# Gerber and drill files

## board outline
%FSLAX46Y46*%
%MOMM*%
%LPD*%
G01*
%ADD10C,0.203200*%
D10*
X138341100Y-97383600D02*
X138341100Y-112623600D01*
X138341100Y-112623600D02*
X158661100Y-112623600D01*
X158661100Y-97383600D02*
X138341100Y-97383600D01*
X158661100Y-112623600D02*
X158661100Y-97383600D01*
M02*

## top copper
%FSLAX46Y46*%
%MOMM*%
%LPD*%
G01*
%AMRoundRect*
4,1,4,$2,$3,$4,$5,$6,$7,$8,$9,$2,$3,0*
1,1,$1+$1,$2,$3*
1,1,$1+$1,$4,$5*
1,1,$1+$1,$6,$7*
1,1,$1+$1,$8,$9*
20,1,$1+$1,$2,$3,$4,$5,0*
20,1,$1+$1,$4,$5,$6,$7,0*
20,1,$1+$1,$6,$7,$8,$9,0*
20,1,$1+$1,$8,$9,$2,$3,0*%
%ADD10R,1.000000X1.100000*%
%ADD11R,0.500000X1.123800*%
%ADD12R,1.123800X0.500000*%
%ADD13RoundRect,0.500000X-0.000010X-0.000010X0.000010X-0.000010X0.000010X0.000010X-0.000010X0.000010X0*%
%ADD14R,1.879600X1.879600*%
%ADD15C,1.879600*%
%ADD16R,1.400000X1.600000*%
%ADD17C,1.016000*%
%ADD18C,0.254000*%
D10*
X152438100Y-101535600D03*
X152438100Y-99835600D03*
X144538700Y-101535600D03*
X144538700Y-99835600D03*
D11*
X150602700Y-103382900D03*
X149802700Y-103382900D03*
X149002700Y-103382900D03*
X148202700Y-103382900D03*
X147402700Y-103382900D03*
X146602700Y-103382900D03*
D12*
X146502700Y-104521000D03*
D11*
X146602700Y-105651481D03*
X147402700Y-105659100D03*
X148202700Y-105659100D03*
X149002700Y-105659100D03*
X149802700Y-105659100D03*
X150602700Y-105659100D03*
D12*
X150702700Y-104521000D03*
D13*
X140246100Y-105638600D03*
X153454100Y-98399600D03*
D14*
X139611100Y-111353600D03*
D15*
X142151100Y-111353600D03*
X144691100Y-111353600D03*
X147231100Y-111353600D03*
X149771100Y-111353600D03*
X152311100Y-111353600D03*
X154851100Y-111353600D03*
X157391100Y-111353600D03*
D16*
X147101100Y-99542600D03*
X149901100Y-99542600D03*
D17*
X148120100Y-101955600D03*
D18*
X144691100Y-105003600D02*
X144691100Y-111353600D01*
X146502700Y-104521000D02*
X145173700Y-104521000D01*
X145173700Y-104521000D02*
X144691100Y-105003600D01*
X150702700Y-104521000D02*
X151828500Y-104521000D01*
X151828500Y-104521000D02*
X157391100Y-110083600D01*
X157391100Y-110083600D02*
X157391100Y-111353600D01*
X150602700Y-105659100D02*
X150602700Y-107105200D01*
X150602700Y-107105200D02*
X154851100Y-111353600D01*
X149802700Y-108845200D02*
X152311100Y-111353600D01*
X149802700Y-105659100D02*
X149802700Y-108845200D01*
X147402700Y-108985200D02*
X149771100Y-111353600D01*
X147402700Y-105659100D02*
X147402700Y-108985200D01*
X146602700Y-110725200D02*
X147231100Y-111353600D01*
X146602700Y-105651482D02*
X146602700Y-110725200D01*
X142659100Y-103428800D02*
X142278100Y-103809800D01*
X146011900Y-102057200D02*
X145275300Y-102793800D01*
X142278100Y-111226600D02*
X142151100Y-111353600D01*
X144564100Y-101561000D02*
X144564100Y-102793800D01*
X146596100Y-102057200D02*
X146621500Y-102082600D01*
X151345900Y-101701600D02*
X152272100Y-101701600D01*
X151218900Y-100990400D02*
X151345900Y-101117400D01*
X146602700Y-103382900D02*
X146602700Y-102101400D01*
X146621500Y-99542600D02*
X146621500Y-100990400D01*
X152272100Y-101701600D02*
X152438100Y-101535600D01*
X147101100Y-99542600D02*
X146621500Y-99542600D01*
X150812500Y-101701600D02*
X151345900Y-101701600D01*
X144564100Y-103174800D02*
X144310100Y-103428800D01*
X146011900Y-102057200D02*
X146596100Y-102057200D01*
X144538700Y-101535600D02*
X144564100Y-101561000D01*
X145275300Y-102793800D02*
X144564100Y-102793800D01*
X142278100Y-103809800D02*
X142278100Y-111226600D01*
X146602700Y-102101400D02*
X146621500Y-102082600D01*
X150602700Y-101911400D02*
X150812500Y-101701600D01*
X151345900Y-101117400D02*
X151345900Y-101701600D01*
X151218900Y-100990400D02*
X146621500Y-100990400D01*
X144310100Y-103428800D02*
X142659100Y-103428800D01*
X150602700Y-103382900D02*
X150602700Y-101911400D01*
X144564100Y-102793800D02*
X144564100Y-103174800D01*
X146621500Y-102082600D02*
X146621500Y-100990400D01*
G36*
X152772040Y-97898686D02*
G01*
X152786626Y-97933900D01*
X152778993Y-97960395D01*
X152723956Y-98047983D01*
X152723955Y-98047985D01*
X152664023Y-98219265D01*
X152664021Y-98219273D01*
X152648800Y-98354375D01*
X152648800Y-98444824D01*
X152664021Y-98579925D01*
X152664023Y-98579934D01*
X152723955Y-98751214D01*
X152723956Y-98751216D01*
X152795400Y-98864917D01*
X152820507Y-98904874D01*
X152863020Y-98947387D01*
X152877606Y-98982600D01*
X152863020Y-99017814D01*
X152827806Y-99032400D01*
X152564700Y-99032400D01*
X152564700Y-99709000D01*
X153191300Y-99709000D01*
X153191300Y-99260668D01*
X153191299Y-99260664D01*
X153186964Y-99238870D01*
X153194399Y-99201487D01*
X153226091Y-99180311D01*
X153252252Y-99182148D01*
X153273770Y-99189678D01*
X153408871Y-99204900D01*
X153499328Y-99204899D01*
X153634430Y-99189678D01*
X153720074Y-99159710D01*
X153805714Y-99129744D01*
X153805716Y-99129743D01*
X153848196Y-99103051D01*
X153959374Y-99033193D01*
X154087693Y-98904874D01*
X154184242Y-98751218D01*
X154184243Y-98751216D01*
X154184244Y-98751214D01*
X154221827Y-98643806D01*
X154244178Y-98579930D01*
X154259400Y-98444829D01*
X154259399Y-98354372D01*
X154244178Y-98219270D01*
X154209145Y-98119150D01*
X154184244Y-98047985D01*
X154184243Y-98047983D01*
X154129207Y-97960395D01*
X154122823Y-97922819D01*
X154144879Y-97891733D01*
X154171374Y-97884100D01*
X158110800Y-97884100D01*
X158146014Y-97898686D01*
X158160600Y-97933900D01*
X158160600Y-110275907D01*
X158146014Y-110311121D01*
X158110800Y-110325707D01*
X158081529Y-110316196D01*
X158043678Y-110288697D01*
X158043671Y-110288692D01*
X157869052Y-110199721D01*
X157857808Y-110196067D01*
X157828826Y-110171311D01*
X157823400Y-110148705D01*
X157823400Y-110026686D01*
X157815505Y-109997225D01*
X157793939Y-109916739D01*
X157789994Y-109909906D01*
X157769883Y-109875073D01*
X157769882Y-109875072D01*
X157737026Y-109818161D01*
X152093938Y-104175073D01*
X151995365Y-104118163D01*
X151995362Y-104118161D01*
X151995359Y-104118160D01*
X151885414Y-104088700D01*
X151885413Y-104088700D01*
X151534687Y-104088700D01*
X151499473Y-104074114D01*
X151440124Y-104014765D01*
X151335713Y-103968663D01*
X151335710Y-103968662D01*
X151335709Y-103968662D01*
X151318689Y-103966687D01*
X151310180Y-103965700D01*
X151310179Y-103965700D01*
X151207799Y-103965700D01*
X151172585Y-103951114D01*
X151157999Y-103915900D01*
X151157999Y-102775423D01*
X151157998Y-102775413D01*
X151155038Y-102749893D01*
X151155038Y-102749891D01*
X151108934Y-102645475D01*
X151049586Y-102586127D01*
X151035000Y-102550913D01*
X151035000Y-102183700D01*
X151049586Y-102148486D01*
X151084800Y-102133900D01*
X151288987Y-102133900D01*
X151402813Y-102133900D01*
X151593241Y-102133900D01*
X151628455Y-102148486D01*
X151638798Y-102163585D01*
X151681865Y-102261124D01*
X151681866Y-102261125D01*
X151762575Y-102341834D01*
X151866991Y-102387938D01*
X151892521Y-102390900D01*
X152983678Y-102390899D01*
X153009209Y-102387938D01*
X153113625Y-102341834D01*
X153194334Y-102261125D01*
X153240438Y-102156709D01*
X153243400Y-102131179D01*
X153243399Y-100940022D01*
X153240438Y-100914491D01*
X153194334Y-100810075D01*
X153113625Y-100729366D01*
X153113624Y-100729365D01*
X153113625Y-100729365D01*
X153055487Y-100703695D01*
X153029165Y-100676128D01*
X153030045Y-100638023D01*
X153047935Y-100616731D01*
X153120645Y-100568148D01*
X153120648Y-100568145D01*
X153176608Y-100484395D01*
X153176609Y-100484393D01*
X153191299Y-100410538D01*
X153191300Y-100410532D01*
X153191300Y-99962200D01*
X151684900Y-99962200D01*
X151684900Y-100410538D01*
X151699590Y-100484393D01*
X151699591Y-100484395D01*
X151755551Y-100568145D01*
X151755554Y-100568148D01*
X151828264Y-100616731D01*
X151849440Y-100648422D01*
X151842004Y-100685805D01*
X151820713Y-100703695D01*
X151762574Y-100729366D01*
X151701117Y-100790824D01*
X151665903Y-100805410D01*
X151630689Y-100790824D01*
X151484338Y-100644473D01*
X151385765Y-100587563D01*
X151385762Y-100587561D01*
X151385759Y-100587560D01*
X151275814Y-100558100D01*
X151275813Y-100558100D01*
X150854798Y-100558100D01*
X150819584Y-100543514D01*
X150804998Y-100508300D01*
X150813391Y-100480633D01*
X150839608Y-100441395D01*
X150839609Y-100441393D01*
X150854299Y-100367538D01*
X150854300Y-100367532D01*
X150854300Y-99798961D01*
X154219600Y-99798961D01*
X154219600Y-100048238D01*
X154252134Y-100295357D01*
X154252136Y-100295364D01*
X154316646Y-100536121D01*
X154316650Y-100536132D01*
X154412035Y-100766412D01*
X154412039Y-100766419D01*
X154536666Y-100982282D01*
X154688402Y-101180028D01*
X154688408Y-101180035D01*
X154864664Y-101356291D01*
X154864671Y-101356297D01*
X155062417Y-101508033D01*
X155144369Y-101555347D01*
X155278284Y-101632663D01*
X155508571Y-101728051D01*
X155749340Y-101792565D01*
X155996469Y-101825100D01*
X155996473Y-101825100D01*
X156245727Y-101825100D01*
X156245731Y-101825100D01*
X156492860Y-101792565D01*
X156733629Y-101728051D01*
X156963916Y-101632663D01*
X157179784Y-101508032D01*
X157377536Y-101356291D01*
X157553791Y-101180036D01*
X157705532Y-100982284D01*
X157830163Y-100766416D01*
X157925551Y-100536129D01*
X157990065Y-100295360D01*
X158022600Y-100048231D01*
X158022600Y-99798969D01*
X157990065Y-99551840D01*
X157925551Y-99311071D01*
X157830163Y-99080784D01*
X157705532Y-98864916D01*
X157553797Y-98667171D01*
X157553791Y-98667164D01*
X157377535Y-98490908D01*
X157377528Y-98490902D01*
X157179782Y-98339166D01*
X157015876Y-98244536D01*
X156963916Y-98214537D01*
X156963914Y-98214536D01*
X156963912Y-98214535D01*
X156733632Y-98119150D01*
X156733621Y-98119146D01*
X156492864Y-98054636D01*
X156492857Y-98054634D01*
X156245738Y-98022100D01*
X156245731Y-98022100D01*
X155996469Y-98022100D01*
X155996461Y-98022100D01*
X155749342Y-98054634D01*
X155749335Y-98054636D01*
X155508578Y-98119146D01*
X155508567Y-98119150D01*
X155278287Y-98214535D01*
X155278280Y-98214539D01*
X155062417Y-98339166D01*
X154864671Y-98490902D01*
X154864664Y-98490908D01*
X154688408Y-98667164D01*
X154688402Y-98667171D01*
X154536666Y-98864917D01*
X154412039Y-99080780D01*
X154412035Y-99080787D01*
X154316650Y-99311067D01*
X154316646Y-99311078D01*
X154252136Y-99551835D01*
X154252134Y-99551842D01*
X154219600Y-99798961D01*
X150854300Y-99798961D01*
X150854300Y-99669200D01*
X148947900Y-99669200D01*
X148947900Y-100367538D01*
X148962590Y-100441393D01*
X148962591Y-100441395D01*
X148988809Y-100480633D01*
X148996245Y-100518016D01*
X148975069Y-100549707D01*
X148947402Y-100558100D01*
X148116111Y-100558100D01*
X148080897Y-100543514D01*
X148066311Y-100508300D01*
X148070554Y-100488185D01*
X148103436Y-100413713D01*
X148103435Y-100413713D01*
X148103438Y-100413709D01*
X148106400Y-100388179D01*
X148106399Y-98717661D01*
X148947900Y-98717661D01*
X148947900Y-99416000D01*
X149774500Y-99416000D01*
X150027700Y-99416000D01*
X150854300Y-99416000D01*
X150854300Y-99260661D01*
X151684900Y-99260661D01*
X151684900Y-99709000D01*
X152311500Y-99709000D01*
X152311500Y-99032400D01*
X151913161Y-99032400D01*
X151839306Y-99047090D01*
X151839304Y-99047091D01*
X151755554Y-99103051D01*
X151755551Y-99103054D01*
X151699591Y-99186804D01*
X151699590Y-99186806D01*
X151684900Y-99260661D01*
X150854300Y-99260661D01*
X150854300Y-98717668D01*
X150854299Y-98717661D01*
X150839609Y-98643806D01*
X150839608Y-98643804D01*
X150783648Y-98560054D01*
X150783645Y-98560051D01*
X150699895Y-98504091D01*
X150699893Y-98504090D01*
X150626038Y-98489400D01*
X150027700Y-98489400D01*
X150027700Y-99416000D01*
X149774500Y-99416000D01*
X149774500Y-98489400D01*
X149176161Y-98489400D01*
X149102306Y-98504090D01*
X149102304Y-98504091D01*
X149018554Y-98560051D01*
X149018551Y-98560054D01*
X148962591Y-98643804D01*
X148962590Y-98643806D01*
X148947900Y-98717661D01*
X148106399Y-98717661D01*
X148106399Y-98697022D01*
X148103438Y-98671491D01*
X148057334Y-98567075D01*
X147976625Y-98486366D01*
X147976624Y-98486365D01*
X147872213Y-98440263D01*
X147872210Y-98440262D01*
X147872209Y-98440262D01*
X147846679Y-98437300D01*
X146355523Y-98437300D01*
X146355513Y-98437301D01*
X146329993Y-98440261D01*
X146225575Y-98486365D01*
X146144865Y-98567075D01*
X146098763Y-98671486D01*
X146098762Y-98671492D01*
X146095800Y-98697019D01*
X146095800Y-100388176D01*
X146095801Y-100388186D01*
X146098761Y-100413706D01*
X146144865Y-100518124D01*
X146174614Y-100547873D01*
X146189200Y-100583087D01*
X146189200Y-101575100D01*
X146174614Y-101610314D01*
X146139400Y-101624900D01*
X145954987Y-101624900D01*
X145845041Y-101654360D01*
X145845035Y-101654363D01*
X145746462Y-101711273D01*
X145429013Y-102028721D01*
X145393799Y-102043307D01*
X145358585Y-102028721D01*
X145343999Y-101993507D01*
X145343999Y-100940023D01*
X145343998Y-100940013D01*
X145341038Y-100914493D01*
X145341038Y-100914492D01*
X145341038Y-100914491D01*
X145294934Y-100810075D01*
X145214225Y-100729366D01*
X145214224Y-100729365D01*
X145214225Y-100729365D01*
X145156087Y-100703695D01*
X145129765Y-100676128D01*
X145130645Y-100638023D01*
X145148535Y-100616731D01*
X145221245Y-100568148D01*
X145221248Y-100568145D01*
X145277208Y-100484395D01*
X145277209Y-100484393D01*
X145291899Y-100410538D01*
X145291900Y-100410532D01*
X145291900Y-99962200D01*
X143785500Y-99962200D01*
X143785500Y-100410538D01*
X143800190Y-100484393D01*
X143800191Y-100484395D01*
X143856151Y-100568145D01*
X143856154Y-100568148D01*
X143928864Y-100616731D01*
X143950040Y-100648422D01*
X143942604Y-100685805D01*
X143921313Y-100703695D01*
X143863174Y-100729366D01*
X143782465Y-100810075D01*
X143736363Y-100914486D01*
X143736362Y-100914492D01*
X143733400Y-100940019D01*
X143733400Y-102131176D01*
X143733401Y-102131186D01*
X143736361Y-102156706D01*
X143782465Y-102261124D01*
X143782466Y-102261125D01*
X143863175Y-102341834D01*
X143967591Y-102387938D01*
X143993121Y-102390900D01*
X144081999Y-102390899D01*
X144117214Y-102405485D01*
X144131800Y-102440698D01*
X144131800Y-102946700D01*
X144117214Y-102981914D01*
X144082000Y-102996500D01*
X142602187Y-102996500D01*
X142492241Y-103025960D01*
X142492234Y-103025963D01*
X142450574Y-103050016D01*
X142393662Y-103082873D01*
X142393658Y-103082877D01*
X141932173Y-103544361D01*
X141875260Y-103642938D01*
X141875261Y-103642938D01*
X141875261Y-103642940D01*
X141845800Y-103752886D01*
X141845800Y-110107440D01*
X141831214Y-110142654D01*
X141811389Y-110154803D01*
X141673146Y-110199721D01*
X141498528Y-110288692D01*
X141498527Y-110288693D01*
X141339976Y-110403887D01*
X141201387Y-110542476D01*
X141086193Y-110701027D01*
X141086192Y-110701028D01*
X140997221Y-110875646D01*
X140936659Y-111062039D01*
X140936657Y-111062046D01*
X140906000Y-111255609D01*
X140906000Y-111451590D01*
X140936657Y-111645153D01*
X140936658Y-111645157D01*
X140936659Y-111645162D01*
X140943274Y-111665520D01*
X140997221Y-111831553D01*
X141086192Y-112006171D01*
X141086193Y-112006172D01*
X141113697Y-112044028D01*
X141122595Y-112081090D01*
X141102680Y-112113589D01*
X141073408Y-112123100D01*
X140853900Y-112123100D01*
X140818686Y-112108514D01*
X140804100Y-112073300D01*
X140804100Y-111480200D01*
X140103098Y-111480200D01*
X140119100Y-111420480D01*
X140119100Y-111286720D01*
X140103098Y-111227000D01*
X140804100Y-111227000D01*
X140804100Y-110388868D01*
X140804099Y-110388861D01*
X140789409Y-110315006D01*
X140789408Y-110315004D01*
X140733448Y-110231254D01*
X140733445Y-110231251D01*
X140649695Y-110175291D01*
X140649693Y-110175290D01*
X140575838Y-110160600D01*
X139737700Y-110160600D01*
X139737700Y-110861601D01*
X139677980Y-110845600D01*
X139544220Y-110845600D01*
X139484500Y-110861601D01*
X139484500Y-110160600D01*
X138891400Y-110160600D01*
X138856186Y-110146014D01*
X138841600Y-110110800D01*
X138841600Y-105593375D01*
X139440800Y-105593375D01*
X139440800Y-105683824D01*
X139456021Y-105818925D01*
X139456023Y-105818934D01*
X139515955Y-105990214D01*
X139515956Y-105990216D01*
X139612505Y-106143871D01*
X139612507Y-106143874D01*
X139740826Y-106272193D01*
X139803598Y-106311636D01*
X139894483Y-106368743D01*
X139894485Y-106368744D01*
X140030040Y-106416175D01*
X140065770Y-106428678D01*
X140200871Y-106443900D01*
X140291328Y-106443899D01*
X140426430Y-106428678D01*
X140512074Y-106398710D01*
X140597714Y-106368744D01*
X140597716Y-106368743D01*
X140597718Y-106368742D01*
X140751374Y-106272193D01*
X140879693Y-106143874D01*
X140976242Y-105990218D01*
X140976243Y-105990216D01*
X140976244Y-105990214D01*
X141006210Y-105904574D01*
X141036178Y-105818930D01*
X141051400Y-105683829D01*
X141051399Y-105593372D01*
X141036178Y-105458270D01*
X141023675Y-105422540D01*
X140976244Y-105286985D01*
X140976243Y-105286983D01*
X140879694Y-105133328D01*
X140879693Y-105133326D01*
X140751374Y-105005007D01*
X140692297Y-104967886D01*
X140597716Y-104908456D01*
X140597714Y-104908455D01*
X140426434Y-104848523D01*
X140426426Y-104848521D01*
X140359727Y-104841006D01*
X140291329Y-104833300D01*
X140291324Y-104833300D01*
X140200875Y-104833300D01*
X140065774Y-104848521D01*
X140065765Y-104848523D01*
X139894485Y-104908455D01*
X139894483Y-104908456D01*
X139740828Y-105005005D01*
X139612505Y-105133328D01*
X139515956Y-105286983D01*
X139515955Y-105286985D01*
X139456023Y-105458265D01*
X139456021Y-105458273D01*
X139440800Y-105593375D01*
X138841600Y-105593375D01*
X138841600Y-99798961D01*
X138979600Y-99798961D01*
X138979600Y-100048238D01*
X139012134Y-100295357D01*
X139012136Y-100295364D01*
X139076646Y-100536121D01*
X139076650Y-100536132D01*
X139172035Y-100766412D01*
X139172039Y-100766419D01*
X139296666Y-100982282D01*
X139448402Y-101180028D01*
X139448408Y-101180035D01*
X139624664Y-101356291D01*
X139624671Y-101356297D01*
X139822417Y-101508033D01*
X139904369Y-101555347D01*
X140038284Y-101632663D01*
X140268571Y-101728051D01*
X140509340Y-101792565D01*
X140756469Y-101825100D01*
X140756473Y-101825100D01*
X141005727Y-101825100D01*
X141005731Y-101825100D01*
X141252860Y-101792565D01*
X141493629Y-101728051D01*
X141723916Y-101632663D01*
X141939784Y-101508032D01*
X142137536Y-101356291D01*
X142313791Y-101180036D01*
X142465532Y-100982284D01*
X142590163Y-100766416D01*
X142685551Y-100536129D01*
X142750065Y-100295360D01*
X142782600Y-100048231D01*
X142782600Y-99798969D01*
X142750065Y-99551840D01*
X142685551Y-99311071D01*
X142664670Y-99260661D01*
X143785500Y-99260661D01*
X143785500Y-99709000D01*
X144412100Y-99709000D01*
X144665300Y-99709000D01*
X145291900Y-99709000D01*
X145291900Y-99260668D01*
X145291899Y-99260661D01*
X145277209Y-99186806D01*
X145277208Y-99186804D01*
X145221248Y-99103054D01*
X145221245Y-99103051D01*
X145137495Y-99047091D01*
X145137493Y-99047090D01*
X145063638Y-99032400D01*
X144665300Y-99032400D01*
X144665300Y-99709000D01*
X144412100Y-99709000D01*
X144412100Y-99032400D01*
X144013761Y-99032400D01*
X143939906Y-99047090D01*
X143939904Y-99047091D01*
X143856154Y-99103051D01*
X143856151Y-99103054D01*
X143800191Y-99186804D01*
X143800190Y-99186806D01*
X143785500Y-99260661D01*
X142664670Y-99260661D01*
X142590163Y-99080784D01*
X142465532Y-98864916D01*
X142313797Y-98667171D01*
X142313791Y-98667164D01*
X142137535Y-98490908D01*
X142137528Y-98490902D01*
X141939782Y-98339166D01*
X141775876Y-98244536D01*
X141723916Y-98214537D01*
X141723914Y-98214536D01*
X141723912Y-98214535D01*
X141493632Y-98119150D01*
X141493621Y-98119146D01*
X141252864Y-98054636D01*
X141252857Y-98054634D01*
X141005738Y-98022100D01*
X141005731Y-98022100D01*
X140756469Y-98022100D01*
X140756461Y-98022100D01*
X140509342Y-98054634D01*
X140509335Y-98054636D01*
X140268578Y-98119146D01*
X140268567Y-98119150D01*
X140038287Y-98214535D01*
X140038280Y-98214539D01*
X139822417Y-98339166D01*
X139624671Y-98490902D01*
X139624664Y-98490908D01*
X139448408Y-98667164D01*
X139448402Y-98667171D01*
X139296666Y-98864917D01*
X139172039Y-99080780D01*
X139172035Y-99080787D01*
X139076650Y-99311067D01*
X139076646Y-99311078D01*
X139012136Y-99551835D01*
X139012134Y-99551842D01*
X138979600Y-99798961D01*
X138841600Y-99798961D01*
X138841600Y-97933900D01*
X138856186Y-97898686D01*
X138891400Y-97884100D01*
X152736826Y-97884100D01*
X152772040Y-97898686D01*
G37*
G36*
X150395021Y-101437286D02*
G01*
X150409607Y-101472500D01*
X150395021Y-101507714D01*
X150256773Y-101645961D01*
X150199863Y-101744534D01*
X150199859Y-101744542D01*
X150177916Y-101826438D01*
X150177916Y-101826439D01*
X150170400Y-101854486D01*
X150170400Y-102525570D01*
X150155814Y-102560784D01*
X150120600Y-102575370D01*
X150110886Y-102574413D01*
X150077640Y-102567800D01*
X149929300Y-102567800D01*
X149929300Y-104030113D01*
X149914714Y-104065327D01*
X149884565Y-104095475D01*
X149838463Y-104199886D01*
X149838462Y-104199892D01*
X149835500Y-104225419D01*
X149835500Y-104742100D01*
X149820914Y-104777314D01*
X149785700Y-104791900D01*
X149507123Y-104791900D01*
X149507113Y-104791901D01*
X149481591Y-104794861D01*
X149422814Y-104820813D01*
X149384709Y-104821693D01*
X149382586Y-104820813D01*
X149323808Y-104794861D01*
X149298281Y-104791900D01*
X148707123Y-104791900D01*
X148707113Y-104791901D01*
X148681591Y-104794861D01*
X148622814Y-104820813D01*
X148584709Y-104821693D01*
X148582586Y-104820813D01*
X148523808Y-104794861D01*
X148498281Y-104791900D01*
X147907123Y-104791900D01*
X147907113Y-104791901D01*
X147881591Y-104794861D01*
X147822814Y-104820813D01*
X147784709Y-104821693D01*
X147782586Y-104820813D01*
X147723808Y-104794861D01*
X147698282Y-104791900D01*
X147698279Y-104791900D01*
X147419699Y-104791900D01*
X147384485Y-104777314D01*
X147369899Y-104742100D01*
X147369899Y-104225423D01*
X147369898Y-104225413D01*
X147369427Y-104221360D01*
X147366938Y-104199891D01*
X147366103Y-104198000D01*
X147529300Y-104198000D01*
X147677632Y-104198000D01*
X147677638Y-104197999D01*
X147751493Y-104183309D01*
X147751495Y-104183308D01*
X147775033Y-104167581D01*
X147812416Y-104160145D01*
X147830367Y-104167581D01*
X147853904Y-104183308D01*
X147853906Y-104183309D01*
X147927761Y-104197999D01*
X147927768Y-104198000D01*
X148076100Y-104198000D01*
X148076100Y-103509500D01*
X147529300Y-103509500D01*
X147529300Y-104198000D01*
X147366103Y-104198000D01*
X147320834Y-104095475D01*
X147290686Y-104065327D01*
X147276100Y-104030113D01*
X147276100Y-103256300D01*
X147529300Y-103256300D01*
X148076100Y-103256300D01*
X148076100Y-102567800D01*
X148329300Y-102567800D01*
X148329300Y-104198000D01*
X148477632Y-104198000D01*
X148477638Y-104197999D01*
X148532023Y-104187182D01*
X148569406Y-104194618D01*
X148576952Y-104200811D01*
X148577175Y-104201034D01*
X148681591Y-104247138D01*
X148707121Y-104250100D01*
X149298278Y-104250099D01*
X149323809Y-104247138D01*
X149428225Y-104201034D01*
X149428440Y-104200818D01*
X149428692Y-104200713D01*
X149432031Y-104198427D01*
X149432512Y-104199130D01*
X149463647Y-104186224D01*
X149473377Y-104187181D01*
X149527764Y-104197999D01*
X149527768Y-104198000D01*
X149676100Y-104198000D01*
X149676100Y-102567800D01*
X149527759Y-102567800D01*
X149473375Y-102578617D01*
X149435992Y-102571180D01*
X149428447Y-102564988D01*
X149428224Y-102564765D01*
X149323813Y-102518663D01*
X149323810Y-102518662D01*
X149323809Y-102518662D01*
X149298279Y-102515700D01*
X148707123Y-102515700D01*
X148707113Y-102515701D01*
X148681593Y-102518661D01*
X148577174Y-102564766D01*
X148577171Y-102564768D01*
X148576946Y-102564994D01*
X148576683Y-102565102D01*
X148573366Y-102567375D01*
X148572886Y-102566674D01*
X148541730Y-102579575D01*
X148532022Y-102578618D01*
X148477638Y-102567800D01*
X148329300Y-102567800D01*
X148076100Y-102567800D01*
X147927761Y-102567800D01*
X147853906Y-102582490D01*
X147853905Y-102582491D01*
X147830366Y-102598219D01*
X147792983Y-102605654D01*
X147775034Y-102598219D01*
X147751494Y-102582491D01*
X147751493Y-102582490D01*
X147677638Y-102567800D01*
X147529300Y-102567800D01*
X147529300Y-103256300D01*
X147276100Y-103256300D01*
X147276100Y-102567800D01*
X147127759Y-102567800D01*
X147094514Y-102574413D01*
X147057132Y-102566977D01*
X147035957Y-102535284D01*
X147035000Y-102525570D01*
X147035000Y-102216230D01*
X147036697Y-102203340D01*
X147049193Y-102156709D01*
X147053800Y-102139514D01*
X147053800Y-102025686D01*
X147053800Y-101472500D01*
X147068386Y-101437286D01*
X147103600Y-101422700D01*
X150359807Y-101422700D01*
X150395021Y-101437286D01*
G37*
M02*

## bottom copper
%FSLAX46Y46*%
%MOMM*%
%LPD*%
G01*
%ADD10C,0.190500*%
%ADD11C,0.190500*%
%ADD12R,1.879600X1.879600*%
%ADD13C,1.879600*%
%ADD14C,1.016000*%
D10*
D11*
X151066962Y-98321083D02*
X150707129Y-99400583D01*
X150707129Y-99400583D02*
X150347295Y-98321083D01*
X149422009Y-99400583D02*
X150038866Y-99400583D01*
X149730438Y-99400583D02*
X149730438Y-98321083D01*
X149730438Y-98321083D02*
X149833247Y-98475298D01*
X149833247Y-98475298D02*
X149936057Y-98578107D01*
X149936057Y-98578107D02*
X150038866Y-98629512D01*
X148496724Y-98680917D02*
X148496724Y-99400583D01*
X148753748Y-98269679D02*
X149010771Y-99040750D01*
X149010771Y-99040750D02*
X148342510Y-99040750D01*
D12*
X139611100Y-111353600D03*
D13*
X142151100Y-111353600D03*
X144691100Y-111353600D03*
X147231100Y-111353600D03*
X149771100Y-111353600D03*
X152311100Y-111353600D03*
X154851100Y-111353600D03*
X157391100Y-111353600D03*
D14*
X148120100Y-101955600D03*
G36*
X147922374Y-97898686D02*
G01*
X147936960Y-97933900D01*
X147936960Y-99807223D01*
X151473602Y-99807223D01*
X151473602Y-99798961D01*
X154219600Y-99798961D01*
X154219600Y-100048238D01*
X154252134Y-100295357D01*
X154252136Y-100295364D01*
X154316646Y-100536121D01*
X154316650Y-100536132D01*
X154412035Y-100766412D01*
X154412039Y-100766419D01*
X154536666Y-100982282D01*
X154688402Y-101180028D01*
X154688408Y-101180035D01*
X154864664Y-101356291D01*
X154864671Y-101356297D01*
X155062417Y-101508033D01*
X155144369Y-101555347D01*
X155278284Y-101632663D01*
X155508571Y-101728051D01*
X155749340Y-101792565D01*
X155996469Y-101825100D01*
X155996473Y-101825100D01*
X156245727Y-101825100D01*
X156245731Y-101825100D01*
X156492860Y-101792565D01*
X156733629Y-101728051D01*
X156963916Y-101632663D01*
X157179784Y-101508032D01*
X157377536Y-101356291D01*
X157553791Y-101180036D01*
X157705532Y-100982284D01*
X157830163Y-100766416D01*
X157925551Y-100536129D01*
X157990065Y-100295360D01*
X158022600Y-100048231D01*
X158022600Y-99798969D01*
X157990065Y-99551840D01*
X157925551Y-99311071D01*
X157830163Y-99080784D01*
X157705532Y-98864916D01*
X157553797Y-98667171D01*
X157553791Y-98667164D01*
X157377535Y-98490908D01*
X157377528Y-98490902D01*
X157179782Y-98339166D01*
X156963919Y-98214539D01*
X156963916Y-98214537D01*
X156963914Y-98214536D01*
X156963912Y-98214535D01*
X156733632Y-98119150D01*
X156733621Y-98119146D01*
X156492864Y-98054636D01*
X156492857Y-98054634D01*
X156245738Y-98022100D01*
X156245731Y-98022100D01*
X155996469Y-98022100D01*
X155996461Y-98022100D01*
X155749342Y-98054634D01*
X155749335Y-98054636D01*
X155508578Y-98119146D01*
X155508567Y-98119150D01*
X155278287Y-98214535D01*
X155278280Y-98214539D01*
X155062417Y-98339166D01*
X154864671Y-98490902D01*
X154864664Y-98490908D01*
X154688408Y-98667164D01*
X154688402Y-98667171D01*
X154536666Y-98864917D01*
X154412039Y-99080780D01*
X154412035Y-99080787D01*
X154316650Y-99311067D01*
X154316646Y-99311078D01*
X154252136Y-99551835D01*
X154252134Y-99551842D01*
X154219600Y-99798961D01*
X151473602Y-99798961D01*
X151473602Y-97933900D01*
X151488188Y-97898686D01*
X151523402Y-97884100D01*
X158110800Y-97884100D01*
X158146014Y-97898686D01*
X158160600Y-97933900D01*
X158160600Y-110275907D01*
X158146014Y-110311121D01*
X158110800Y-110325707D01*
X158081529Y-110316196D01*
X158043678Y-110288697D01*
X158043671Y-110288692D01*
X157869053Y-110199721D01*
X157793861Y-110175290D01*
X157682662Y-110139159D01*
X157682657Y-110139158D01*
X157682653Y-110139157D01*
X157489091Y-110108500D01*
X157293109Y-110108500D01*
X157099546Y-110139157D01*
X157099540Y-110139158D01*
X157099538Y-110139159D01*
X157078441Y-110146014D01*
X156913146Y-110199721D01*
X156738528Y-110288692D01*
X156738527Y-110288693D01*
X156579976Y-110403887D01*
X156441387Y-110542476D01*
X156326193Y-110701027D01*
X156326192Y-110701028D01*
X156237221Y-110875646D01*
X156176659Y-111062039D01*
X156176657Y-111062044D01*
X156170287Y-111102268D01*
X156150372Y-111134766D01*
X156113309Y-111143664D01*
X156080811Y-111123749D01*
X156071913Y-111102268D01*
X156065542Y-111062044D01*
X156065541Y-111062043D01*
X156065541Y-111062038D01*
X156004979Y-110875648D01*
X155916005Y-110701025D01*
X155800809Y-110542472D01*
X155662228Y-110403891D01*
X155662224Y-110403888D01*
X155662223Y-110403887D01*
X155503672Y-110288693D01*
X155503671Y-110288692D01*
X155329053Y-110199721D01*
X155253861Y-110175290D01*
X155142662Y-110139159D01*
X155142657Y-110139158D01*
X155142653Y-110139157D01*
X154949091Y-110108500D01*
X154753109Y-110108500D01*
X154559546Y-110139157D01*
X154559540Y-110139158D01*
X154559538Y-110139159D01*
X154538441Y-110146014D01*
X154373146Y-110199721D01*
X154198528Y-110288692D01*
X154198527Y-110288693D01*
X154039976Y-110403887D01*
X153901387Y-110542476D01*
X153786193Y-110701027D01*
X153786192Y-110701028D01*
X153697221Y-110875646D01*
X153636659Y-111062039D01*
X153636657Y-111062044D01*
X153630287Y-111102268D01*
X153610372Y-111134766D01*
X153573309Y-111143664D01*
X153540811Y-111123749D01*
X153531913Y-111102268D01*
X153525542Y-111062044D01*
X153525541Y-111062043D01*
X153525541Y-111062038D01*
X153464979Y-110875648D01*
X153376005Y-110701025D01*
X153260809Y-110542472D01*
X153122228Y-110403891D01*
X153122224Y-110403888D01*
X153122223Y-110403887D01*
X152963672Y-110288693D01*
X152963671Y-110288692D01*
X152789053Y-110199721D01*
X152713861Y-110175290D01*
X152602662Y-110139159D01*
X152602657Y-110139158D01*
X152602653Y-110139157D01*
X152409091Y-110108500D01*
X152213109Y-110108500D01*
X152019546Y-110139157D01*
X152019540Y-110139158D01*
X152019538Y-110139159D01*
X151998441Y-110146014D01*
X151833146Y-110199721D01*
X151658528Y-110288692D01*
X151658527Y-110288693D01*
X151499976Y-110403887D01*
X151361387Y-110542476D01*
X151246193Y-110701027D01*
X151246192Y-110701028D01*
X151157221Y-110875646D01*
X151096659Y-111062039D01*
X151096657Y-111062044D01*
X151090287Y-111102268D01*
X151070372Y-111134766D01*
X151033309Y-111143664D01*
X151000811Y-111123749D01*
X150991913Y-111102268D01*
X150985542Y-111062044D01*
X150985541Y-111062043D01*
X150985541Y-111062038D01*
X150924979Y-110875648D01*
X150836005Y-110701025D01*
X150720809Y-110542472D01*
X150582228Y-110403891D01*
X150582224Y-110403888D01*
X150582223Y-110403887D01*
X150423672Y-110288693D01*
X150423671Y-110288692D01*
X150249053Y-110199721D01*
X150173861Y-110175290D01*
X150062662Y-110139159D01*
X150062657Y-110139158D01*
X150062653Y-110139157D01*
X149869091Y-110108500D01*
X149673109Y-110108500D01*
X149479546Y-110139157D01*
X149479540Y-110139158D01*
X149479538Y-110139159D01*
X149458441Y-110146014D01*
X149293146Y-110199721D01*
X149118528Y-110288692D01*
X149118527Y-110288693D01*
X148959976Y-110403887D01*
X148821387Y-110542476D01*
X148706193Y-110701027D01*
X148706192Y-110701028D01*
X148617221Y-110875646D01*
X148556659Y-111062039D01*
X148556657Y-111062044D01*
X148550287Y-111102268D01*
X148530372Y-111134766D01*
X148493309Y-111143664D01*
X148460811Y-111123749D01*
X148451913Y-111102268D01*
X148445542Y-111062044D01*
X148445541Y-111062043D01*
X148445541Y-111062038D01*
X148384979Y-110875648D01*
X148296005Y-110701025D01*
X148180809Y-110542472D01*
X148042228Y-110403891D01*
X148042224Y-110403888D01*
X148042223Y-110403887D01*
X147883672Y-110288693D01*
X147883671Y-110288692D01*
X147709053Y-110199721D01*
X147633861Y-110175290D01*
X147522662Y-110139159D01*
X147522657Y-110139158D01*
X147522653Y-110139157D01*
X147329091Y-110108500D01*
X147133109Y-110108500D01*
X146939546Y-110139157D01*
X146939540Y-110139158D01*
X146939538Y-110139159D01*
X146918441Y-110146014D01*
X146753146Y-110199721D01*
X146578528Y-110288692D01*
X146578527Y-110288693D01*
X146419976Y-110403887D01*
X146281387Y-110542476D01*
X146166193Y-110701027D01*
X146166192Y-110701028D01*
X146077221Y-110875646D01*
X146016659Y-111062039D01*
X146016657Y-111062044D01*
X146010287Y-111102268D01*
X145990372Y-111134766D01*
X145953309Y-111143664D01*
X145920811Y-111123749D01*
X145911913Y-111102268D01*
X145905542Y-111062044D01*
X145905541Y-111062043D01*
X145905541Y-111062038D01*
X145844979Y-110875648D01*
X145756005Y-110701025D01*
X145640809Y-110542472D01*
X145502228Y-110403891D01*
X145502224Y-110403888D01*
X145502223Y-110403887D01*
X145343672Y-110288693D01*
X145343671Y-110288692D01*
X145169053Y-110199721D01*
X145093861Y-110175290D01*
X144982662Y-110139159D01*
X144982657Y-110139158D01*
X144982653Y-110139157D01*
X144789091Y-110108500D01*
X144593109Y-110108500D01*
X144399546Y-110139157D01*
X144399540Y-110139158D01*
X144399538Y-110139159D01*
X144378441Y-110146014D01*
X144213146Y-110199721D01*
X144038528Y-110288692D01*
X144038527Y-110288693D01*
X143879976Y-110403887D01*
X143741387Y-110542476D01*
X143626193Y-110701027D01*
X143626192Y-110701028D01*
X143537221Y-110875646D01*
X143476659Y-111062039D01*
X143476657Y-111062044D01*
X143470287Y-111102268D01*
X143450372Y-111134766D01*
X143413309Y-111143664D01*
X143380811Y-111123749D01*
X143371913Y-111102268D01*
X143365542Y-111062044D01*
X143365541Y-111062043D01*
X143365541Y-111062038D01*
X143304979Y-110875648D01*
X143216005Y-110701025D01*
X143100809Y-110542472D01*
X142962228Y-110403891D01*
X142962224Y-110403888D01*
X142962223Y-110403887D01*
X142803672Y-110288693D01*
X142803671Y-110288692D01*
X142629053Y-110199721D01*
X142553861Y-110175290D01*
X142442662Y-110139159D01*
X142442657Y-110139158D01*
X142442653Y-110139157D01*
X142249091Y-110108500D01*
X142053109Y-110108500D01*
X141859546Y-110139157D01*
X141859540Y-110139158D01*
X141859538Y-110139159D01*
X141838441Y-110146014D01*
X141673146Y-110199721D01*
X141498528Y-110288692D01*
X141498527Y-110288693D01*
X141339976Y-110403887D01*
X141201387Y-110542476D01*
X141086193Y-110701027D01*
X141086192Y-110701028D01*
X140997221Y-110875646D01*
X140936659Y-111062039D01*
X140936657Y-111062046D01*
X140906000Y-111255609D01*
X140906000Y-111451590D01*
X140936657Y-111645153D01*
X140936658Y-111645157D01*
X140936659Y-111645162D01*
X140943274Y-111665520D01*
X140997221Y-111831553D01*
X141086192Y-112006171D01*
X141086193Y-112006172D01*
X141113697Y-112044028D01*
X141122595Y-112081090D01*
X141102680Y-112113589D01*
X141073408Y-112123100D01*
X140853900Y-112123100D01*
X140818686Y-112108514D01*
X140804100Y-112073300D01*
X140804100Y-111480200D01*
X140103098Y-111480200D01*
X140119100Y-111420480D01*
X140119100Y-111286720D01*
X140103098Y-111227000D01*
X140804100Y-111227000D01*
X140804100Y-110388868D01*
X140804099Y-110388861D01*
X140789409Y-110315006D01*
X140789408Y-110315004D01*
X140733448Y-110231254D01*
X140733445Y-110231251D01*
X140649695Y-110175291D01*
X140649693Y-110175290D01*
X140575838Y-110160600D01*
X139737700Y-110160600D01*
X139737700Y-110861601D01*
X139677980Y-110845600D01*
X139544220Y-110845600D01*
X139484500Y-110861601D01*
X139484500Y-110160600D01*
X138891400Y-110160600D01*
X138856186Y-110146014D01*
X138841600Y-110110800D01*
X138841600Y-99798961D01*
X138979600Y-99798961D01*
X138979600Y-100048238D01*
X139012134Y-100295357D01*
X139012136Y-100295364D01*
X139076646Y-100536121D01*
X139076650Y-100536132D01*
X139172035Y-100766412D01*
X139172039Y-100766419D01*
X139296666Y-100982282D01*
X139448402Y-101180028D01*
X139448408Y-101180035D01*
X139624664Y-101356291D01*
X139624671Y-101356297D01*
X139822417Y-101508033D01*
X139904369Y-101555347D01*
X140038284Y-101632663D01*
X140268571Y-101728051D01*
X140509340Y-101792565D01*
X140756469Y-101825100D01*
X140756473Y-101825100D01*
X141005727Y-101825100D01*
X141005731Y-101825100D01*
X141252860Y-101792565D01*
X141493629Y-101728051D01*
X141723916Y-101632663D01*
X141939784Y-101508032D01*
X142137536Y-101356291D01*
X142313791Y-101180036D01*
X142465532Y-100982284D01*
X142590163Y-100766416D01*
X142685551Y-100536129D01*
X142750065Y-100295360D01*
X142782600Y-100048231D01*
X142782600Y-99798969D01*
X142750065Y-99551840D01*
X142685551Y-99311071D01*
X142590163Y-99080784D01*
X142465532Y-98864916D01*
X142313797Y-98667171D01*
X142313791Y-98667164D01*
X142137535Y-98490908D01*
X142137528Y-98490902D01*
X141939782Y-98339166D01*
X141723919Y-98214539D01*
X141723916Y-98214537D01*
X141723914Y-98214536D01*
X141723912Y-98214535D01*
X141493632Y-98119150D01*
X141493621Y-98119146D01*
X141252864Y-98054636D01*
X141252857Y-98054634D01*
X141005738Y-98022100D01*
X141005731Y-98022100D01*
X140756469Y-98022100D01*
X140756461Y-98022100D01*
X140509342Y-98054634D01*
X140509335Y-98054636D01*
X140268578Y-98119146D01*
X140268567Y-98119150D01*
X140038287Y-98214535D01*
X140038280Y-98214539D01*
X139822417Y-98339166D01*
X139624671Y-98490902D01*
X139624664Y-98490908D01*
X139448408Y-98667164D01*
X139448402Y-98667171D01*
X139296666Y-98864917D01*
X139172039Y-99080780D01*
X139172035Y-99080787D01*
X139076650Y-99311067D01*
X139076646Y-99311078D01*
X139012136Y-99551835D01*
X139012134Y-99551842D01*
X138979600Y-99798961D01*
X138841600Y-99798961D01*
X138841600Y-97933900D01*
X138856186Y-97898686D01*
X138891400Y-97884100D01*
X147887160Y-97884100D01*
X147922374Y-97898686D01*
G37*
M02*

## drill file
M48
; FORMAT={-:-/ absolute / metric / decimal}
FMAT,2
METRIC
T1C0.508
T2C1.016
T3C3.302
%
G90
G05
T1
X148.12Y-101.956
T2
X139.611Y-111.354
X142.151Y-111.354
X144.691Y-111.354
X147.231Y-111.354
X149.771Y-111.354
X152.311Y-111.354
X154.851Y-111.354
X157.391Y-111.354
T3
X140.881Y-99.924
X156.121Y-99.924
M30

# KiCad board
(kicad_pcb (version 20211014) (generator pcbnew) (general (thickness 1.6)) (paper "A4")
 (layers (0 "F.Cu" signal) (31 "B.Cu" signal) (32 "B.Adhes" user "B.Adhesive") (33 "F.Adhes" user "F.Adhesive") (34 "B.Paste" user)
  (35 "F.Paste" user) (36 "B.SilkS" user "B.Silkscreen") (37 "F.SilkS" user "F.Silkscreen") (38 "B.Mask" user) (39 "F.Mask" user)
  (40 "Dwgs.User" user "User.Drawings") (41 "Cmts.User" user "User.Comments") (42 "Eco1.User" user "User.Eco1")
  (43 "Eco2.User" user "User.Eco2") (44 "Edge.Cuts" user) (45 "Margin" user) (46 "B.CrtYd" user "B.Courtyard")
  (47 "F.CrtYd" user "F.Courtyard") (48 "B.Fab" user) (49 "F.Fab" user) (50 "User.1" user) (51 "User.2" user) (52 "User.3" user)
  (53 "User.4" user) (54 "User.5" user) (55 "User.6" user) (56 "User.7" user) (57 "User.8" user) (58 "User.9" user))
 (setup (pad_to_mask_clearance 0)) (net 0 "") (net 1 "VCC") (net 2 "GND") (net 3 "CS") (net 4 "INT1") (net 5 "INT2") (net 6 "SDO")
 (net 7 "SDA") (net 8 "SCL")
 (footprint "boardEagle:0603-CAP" (layer "F.Cu") (at 152.4381 100.6856 90)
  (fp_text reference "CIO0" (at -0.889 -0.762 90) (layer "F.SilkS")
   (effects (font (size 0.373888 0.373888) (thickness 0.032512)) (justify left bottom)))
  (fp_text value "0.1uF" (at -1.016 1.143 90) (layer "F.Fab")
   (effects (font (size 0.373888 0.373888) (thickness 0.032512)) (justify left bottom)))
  (pad "1" smd rect (at -0.85 0 90) (size 1.1 1) (layers "F.Cu" "F.Paste" "F.Mask") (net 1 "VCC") (solder_mask_margin 0.1016))
  (pad "2" smd rect (at 0.85 0 90) (size 1.1 1) (layers "F.Cu" "F.Paste" "F.Mask") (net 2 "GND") (solder_mask_margin 0.1016)))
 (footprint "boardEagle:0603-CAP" (layer "F.Cu") (at 144.5387 100.6856 90)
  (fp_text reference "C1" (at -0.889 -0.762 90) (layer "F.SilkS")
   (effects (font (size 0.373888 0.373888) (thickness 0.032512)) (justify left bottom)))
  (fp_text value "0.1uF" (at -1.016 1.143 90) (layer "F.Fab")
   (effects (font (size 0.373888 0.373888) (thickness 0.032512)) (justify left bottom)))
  (pad "1" smd rect (at -0.85 0 90) (size 1.1 1) (layers "F.Cu" "F.Paste" "F.Mask") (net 1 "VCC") (solder_mask_margin 0.1016))
  (pad "2" smd rect (at 0.85 0 90) (size 1.1 1) (layers "F.Cu" "F.Paste" "F.Mask") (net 2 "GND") (solder_mask_margin 0.1016)))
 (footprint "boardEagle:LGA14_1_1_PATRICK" (layer "F.Cu") (at 148.6027 104.521)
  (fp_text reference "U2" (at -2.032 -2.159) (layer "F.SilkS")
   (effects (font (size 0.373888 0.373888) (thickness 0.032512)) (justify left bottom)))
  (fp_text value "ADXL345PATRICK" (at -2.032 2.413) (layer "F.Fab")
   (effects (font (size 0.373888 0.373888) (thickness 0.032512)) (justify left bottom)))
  (pad "1" smd rect (at 2 -1.1381) (size 0.5 1.1238) (layers "F.Cu" "F.Paste" "F.Mask") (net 1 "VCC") (solder_mask_margin 0.1016))
  (pad "2" smd rect (at 1.2 -1.1381 180) (size 0.5 1.1238) (layers "F.Cu" "F.Paste" "F.Mask") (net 2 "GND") (solder_mask_margin 0.1016))
  (pad "3" smd rect (at 0.4 -1.1381 180) (size 0.5 1.1238) (layers "F.Cu" "F.Paste" "F.Mask") (solder_mask_margin 0.1016))
  (pad "4" smd rect (at -0.4 -1.1381 180) (size 0.5 1.1238) (layers "F.Cu" "F.Paste" "F.Mask") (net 2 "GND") (solder_mask_margin 0.1016))
  (pad "5" smd rect (at -1.2 -1.1381 180) (size 0.5 1.1238) (layers "F.Cu" "F.Paste" "F.Mask") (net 2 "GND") (solder_mask_margin 0.1016))
  (pad "6" smd rect (at -2 -1.1381 180) (size 0.5 1.1238) (layers "F.Cu" "F.Paste" "F.Mask") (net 1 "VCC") (solder_mask_margin 0.1016))
  (pad "7" smd rect (at -2.1 0 270) (size 0.5 1.1238) (layers "F.Cu" "F.Paste" "F.Mask") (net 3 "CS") (solder_mask_margin 0.1016))
  (pad "8" smd rect (at -2 1.130481 180) (size 0.5 1.1238) (layers "F.Cu" "F.Paste" "F.Mask") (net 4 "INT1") (solder_mask_margin 0.1016))
  (pad "9" smd rect (at -1.2 1.1381 180) (size 0.5 1.1238) (layers "F.Cu" "F.Paste" "F.Mask") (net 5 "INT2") (solder_mask_margin 0.1016))
  (pad "10" smd rect (at -0.4 1.1381) (size 0.5 1.1238) (layers "F.Cu" "F.Paste" "F.Mask") (solder_mask_margin 0.1016))
  (pad "11" smd rect (at 0.4 1.1381) (size 0.5 1.1238) (layers "F.Cu" "F.Paste" "F.Mask") (solder_mask_margin 0.1016))
  (pad "12" smd rect (at 1.2 1.1381) (size 0.5 1.1238) (layers "F.Cu" "F.Paste" "F.Mask") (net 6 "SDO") (solder_mask_margin 0.1016))
  (pad "13" smd rect (at 2 1.1381) (size 0.5 1.1238) (layers "F.Cu" "F.Paste" "F.Mask") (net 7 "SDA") (solder_mask_margin 0.1016))
  (pad "14" smd rect (at 2.1 0 90) (size 0.5 1.1238) (layers "F.Cu" "F.Paste" "F.Mask") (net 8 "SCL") (solder_mask_margin 0.1016)))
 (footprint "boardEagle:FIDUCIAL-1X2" (layer "F.Cu") (at 140.2461 105.6386)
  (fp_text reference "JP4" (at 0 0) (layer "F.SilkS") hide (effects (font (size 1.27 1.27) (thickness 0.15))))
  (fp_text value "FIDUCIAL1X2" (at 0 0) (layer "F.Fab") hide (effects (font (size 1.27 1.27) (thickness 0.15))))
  (pad "1" smd roundrect (at 0 0) (size 1 1) (layers "F.Cu" "F.Mask") (roundrect_rratio 0.5) (solder_mask_margin 0.1016)))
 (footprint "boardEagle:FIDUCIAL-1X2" (layer "F.Cu") (at 153.4541 98.3996)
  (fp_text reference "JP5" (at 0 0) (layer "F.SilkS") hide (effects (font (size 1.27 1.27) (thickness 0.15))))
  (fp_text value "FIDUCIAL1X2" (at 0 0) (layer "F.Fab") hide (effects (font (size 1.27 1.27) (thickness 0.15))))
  (pad "1" smd roundrect (at 0 0) (size 1 1) (layers "F.Cu" "F.Mask") (roundrect_rratio 0.5) (solder_mask_margin 0.1016)))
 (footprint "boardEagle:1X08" (layer "F.Cu") (at 139.6111 111.3536)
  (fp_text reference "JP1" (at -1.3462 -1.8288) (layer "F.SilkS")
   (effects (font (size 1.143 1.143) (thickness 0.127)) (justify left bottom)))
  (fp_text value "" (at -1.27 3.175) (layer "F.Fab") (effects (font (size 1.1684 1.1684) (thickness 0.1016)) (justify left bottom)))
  (pad "1" thru_hole rect (at 0 0 90) (size 1.8796 1.8796) (drill 1.016) (layers *.Cu *.Mask) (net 2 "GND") (solder_mask_margin 0.1016))
  (pad "2" thru_hole circle (at 2.54 0 90) (size 1.8796 1.8796) (drill 1.016) (layers *.Cu *.Mask) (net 1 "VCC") (solder_mask_margin 0.1016))
  (pad "3" thru_hole circle (at 5.08 0 90) (size 1.8796 1.8796) (drill 1.016) (layers *.Cu *.Mask) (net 3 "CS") (solder_mask_margin 0.1016))
  (pad "4" thru_hole circle (at 7.62 0 90) (size 1.8796 1.8796) (drill 1.016) (layers *.Cu *.Mask) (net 4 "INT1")
   (solder_mask_margin 0.1016))
  (pad "5" thru_hole circle (at 10.16 0 90) (size 1.8796 1.8796) (drill 1.016) (layers *.Cu *.Mask) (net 5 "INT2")
   (solder_mask_margin 0.1016))
  (pad "6" thru_hole circle (at 12.7 0 90) (size 1.8796 1.8796) (drill 1.016) (layers *.Cu *.Mask) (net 6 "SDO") (solder_mask_margin 0.1016))
  (pad "7" thru_hole circle (at 15.24 0 90) (size 1.8796 1.8796) (drill 1.016) (layers *.Cu *.Mask) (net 7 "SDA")
   (solder_mask_margin 0.1016))
  (pad "8" thru_hole circle (at 17.78 0 90) (size 1.8796 1.8796) (drill 1.016) (layers *.Cu *.Mask) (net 8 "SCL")
   (solder_mask_margin 0.1016)))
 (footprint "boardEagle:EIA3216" (layer "F.Cu") (at 148.5011 99.5426 180)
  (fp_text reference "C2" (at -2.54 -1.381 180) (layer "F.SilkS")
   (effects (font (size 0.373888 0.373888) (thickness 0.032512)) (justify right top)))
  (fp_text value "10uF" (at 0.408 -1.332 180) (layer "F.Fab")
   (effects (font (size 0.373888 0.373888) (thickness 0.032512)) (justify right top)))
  (pad "A" smd rect (at 1.4 0 270) (size 1.6 1.4) (layers "F.Cu" "F.Paste" "F.Mask") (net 1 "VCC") (solder_mask_margin 0.1016))
  (pad "C" smd rect (at -1.4 0 270) (size 1.6 1.4) (layers "F.Cu" "F.Paste" "F.Mask") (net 2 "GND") (solder_mask_margin 0.1016)))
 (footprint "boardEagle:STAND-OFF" (layer "F.Cu") (at 140.8811 99.9236)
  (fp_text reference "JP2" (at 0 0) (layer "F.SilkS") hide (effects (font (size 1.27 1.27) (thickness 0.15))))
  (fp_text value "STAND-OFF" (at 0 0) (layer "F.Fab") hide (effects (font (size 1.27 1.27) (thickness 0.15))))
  (pad "" np_thru_hole circle (at 0 0) (size 3.302 3.302) (drill 3.302) (layers *.Cu *.Mask)))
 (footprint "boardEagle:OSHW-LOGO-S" (layer "F.Cu") (at 144.0307 104.8512)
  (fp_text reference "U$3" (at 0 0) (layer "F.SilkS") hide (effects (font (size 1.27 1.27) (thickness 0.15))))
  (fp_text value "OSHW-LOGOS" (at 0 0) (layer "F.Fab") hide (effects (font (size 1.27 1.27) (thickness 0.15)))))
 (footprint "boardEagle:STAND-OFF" (layer "F.Cu") (at 156.1211 99.9236)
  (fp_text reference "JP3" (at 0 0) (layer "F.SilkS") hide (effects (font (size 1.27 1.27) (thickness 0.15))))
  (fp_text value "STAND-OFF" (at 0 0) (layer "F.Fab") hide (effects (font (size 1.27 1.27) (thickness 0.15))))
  (pad "" np_thru_hole circle (at 0 0) (size 3.302 3.302) (drill 3.302) (layers *.Cu *.Mask)))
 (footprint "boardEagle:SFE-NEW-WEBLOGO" (layer "B.Cu") (at 158.0261 104.7496 180)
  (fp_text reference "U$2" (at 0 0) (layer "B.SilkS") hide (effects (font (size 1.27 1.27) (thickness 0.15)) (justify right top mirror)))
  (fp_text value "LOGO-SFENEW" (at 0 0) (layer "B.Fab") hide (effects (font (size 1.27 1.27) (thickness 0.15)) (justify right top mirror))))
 (gr_line (start 138.3411 97.3836) (end 138.3411 112.6236) (layer "Edge.Cuts") (width 0.2032))
 (gr_line (start 138.3411 112.6236) (end 158.6611 112.6236) (layer "Edge.Cuts") (width 0.2032))
 (gr_line (start 158.6611 97.3836) (end 138.3411 97.3836) (layer "Edge.Cuts") (width 0.2032))
 (gr_line (start 158.6611 112.6236) (end 158.6611 97.3836) (layer "Edge.Cuts") (width 0.2032))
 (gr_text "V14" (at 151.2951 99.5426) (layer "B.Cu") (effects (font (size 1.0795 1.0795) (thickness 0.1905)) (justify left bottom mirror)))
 (via (at 148.1201 101.9556) (size 1.016) (drill 0.508) (layers "F.Cu" "B.Cu") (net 2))
 (segment (start 144.6911 105.0036) (end 144.6911 111.3536) (width 0.254) (layer "F.Cu") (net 3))
 (segment (start 146.5027 104.521) (end 145.1737 104.521) (width 0.254) (layer "F.Cu") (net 3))
 (segment (start 145.1737 104.521) (end 144.6911 105.0036) (width 0.254) (layer "F.Cu") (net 3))
 (segment (start 150.7027 104.521) (end 151.8285 104.521) (width 0.254) (layer "F.Cu") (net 8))
 (segment (start 151.8285 104.521) (end 157.3911 110.0836) (width 0.254) (layer "F.Cu") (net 8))
 (segment (start 157.3911 110.0836) (end 157.3911 111.3536) (width 0.254) (layer "F.Cu") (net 8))
 (segment (start 150.6027 105.6591) (end 150.6027 107.1052) (width 0.254) (layer "F.Cu") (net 7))
 (segment (start 150.6027 107.1052) (end 154.8511 111.3536) (width 0.254) (layer "F.Cu") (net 7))
 (segment (start 149.8027 108.8452) (end 152.3111 111.3536) (width 0.254) (layer "F.Cu") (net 6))
 (segment (start 149.8027 105.6591) (end 149.8027 108.8452) (width 0.254) (layer "F.Cu") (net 6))
 (segment (start 147.4027 108.9852) (end 149.7711 111.3536) (width 0.254) (layer "F.Cu") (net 5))
 (segment (start 147.4027 105.6591) (end 147.4027 108.9852) (width 0.254) (layer "F.Cu") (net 5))
 (segment (start 146.6027 110.7252) (end 147.2311 111.3536) (width 0.254) (layer "F.Cu") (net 4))
 (segment (start 146.6027 105.651482) (end 146.6027 110.7252) (width 0.254) (layer "F.Cu") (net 4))
 (segment (start 142.6591 103.4288) (end 142.2781 103.8098) (width 0.254) (layer "F.Cu") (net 1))
 (segment (start 146.0119 102.0572) (end 145.2753 102.7938) (width 0.254) (layer "F.Cu") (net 1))
 (segment (start 142.2781 111.2266) (end 142.1511 111.3536) (width 0.254) (layer "F.Cu") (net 1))
 (segment (start 144.5641 101.561) (end 144.5641 102.7938) (width 0.254) (layer "F.Cu") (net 1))
 (segment (start 146.5961 102.0572) (end 146.6215 102.0826) (width 0.254) (layer "F.Cu") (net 1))
 (segment (start 151.3459 101.7016) (end 152.2721 101.7016) (width 0.254) (layer "F.Cu") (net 1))
 (segment (start 151.2189 100.9904) (end 151.3459 101.1174) (width 0.254) (layer "F.Cu") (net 1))
 (segment (start 146.6027 103.3829) (end 146.6027 102.1014) (width 0.254) (layer "F.Cu") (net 1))
 (segment (start 146.6215 99.5426) (end 146.6215 100.9904) (width 0.254) (layer "F.Cu") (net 1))
 (segment (start 152.2721 101.7016) (end 152.4381 101.5356) (width 0.254) (layer "F.Cu") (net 1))
 (segment (start 147.1011 99.5426) (end 146.6215 99.5426) (width 0.254) (layer "F.Cu") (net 1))
 (segment (start 150.8125 101.7016) (end 151.3459 101.7016) (width 0.254) (layer "F.Cu") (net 1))
 (segment (start 144.5641 103.1748) (end 144.3101 103.4288) (width 0.254) (layer "F.Cu") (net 1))
 (segment (start 146.0119 102.0572) (end 146.5961 102.0572) (width 0.254) (layer "F.Cu") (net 1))
 (segment (start 144.5387 101.5356) (end 144.5641 101.561) (width 0.254) (layer "F.Cu") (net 1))
 (segment (start 145.2753 102.7938) (end 144.5641 102.7938) (width 0.254) (layer "F.Cu") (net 1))
 (segment (start 142.2781 103.8098) (end 142.2781 111.2266) (width 0.254) (layer "F.Cu") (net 1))
 (segment (start 146.6027 102.1014) (end 146.6215 102.0826) (width 0.254) (layer "F.Cu") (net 1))
 (segment (start 150.6027 101.9114) (end 150.8125 101.7016) (width 0.254) (layer "F.Cu") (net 1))
 (segment (start 151.3459 101.1174) (end 151.3459 101.7016) (width 0.254) (layer "F.Cu") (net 1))
 (segment (start 151.2189 100.9904) (end 146.6215 100.9904) (width 0.254) (layer "F.Cu") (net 1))
 (segment (start 144.3101 103.4288) (end 142.6591 103.4288) (width 0.254) (layer "F.Cu") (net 1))
 (segment (start 150.6027 103.3829) (end 150.6027 101.9114) (width 0.254) (layer "F.Cu") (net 1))
 (segment (start 144.5641 102.7938) (end 144.5641 103.1748) (width 0.254) (layer "F.Cu") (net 1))
 (segment (start 146.6215 102.0826) (end 146.6215 100.9904) (width 0.254) (layer "F.Cu") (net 1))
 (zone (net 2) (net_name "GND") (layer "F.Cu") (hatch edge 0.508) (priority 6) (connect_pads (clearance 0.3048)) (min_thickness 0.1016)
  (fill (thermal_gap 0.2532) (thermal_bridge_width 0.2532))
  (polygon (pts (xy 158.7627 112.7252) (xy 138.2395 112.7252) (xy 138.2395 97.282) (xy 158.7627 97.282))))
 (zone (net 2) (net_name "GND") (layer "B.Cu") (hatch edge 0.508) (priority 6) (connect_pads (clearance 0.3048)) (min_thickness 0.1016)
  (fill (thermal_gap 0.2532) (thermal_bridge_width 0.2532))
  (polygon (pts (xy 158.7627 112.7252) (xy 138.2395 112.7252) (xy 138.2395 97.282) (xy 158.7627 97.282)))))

